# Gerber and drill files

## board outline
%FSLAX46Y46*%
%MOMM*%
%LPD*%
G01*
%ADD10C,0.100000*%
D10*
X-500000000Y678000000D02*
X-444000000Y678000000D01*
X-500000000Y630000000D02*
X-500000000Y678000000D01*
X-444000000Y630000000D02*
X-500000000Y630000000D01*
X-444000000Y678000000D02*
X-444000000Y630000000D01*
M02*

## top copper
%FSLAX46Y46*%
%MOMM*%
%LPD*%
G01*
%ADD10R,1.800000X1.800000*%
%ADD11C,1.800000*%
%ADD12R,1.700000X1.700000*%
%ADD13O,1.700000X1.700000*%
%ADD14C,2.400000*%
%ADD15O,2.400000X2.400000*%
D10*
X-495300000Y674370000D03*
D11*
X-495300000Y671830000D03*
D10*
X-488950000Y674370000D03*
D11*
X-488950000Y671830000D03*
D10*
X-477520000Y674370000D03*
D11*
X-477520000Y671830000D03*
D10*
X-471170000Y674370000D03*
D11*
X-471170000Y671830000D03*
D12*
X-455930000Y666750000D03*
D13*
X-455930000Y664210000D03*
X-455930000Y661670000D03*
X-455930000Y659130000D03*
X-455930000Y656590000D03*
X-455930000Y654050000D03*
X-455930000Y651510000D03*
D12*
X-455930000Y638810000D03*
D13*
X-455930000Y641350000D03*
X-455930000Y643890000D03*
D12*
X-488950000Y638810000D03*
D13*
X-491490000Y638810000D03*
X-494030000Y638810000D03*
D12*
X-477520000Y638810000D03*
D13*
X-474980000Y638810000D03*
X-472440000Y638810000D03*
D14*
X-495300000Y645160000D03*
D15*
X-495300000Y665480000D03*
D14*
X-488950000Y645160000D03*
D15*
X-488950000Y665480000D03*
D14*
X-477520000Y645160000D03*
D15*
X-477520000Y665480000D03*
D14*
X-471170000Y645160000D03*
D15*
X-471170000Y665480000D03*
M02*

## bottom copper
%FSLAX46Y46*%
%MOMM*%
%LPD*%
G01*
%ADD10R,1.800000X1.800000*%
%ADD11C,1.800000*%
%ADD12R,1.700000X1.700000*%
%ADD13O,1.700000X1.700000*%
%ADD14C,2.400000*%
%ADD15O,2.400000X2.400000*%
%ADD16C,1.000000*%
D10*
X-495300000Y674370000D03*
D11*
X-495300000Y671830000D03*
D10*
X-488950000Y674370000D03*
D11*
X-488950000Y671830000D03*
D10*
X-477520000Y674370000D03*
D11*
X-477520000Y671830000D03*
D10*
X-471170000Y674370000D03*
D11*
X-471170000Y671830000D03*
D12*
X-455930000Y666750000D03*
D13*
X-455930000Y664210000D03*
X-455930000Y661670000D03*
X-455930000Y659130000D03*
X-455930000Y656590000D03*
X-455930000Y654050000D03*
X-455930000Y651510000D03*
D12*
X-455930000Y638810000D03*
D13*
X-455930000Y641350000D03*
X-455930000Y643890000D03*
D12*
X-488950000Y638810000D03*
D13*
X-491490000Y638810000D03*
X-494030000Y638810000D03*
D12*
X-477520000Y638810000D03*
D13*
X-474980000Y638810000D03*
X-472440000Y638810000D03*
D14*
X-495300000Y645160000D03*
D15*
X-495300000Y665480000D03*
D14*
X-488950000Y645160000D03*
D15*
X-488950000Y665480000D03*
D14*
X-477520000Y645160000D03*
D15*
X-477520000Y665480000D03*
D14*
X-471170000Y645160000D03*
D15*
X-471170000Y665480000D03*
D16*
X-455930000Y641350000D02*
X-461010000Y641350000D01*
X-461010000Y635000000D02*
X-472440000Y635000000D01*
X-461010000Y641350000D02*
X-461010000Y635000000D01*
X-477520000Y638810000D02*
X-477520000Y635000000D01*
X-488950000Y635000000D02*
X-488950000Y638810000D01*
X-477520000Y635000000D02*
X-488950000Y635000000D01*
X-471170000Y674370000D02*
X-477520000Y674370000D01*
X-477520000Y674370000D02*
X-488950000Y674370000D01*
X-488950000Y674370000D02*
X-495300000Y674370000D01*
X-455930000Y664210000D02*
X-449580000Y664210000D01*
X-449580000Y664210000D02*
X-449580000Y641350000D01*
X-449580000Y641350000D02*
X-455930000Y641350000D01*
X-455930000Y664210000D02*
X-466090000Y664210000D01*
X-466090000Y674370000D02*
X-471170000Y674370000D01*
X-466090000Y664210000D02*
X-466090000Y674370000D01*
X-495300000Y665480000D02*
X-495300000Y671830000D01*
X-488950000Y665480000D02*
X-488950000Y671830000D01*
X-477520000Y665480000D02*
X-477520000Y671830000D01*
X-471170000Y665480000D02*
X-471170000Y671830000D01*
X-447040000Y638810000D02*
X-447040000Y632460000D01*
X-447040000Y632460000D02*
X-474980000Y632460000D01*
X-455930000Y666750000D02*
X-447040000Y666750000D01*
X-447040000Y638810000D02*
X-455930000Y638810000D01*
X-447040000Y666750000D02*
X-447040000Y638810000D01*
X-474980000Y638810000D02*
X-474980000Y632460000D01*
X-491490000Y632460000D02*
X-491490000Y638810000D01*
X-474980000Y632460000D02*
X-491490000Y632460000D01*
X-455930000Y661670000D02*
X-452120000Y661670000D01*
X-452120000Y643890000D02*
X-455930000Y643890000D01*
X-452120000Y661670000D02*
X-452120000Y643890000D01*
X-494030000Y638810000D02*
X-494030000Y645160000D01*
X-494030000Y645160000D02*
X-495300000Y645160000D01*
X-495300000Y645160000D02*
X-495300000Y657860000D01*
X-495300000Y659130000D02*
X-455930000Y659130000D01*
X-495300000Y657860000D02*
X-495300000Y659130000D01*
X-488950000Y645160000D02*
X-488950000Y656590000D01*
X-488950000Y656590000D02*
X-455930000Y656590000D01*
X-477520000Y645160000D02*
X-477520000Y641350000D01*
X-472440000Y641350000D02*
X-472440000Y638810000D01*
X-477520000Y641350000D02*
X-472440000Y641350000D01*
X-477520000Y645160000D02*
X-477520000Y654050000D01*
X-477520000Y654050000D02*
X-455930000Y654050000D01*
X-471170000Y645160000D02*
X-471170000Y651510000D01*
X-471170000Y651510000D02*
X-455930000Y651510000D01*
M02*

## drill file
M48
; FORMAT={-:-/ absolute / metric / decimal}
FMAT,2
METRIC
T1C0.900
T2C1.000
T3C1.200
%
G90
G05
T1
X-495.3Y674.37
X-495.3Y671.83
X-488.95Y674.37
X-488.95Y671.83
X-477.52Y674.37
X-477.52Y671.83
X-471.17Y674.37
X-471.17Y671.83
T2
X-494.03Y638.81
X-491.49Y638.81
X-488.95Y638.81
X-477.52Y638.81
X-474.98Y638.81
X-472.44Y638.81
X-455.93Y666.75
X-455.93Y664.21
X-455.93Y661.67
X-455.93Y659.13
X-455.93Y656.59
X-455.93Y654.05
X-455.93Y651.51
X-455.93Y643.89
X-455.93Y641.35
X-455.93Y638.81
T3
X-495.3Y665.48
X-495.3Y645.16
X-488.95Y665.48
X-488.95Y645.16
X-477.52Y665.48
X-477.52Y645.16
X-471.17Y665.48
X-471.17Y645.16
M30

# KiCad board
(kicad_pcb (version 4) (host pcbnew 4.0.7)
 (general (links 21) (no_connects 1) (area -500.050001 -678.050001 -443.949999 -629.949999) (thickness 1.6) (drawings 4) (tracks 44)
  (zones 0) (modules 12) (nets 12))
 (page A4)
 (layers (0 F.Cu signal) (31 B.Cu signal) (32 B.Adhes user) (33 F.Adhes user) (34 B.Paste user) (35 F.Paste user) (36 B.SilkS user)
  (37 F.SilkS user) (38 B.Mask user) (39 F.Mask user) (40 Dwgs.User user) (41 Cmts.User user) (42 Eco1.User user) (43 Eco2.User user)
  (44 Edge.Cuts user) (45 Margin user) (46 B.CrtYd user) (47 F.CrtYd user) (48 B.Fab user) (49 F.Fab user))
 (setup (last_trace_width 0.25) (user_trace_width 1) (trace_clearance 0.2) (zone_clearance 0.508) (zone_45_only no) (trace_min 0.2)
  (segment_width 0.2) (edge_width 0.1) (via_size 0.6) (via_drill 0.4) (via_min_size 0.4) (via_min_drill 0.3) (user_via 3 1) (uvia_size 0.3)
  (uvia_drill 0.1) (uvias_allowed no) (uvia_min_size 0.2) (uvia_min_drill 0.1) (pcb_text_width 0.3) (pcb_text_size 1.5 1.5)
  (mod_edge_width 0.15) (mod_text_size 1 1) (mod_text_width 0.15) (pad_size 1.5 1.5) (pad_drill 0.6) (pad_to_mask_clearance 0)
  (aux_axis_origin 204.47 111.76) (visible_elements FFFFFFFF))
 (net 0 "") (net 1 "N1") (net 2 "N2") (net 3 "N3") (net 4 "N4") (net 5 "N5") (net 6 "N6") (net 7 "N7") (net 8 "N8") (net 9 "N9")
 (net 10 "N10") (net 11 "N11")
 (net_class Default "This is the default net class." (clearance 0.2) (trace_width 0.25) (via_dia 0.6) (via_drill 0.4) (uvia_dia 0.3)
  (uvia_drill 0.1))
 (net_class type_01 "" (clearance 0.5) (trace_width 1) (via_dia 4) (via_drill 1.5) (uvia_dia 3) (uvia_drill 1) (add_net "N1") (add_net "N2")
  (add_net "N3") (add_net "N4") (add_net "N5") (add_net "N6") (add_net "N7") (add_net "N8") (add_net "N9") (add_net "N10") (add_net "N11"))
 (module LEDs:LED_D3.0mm (layer F.Cu) (at -495.3 -674.37 270)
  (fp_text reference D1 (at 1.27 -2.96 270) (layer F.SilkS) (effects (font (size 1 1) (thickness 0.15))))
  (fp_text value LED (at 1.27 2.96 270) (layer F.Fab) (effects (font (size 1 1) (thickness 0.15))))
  (pad 1 thru_hole rect (at 0 0 270) (size 1.8 1.8) (drill 0.9) (layers *.Cu *.Mask) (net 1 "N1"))
  (pad 2 thru_hole circle (at 2.54 0 270) (size 1.8 1.8) (drill 0.9) (layers *.Cu *.Mask) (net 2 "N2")))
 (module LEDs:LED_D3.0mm (layer F.Cu) (at -488.95 -674.37 270)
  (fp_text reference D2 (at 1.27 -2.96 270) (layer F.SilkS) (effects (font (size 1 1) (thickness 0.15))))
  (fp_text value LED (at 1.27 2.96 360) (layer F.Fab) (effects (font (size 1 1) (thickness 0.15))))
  (pad 1 thru_hole rect (at 0 0 270) (size 1.8 1.8) (drill 0.9) (layers *.Cu *.Mask) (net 1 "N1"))
  (pad 2 thru_hole circle (at 2.54 0 270) (size 1.8 1.8) (drill 0.9) (layers *.Cu *.Mask) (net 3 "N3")))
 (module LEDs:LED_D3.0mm (layer F.Cu) (at -477.52 -674.37 270)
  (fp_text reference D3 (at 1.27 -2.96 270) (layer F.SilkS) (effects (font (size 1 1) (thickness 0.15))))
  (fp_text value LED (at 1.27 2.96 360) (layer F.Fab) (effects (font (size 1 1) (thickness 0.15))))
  (pad 1 thru_hole rect (at 0 0 270) (size 1.8 1.8) (drill 0.9) (layers *.Cu *.Mask) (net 1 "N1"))
  (pad 2 thru_hole circle (at 2.54 0 270) (size 1.8 1.8) (drill 0.9) (layers *.Cu *.Mask) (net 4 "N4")))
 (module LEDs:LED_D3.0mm (layer F.Cu) (at -471.17 -674.37 270)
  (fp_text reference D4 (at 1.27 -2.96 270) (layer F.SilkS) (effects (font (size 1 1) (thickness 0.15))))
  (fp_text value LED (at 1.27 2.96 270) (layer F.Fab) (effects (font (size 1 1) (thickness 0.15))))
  (pad 1 thru_hole rect (at 0 0 270) (size 1.8 1.8) (drill 0.9) (layers *.Cu *.Mask) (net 1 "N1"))
  (pad 2 thru_hole circle (at 2.54 0 270) (size 1.8 1.8) (drill 0.9) (layers *.Cu *.Mask) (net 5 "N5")))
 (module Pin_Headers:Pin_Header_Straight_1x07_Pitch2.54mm (layer F.Cu) (at -455.93 -666.75)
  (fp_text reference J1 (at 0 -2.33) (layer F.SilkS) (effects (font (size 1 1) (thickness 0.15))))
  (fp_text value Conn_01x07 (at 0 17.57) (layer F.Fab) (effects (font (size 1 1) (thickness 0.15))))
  (pad 1 thru_hole rect (at 0 0) (size 1.7 1.7) (drill 1) (layers *.Cu *.Mask) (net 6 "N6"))
  (pad 2 thru_hole oval (at 0 2.54) (size 1.7 1.7) (drill 1) (layers *.Cu *.Mask) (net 1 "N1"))
  (pad 3 thru_hole oval (at 0 5.08) (size 1.7 1.7) (drill 1) (layers *.Cu *.Mask) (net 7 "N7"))
  (pad 4 thru_hole oval (at 0 7.62) (size 1.7 1.7) (drill 1) (layers *.Cu *.Mask) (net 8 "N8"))
  (pad 5 thru_hole oval (at 0 10.16) (size 1.7 1.7) (drill 1) (layers *.Cu *.Mask) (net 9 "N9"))
  (pad 6 thru_hole oval (at 0 12.7) (size 1.7 1.7) (drill 1) (layers *.Cu *.Mask) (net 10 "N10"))
  (pad 7 thru_hole oval (at 0 15.24) (size 1.7 1.7) (drill 1) (layers *.Cu *.Mask) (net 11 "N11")))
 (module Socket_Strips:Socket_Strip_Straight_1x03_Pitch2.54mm (layer F.Cu) (at -455.93 -638.81 180)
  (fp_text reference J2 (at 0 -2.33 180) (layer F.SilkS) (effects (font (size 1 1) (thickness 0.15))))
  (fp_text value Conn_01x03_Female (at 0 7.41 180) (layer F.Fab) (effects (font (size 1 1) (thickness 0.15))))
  (pad 1 thru_hole rect (at 0 0 180) (size 1.7 1.7) (drill 1) (layers *.Cu *.Mask) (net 6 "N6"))
  (pad 2 thru_hole oval (at 0 2.54 180) (size 1.7 1.7) (drill 1) (layers *.Cu *.Mask) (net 1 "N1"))
  (pad 3 thru_hole oval (at 0 5.08 180) (size 1.7 1.7) (drill 1) (layers *.Cu *.Mask) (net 7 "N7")))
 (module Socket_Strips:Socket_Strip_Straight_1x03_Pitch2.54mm (layer F.Cu) (at -488.95 -638.81 270)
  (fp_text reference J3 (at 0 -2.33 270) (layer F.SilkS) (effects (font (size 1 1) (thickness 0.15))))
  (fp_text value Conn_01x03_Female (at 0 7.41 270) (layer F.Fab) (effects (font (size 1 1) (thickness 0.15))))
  (pad 1 thru_hole rect (at 0 0 270) (size 1.7 1.7) (drill 1) (layers *.Cu *.Mask) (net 1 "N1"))
  (pad 2 thru_hole oval (at 0 2.54 270) (size 1.7 1.7) (drill 1) (layers *.Cu *.Mask) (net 6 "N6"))
  (pad 3 thru_hole oval (at 0 5.08 270) (size 1.7 1.7) (drill 1) (layers *.Cu *.Mask) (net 8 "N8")))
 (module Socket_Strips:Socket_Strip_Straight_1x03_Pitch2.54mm (layer F.Cu) (at -477.52 -638.81 90)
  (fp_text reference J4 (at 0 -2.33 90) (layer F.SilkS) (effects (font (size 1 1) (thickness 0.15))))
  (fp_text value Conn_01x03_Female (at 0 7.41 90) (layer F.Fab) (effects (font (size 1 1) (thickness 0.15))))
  (pad 1 thru_hole rect (at 0 0 90) (size 1.7 1.7) (drill 1) (layers *.Cu *.Mask) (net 1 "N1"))
  (pad 2 thru_hole oval (at 0 2.54 90) (size 1.7 1.7) (drill 1) (layers *.Cu *.Mask) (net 6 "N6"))
  (pad 3 thru_hole oval (at 0 5.08 90) (size 1.7 1.7) (drill 1) (layers *.Cu *.Mask) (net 10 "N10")))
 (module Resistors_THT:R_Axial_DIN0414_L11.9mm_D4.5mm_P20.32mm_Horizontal (layer F.Cu) (at -495.3 -645.16 90)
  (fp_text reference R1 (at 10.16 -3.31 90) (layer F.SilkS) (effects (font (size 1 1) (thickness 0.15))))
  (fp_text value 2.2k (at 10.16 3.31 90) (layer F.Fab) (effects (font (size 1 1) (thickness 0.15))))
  (pad 1 thru_hole circle (at 0 0 90) (size 2.4 2.4) (drill 1.2) (layers *.Cu *.Mask) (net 8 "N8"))
  (pad 2 thru_hole oval (at 20.32 0 90) (size 2.4 2.4) (drill 1.2) (layers *.Cu *.Mask) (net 2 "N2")))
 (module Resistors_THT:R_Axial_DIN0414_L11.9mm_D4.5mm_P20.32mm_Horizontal (layer F.Cu) (at -488.95 -645.16 90)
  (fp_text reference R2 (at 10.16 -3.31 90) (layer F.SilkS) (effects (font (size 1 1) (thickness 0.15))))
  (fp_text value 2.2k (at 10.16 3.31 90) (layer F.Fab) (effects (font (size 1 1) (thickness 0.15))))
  (pad 1 thru_hole circle (at 0 0 90) (size 2.4 2.4) (drill 1.2) (layers *.Cu *.Mask) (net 9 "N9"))
  (pad 2 thru_hole oval (at 20.32 0 90) (size 2.4 2.4) (drill 1.2) (layers *.Cu *.Mask) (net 3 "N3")))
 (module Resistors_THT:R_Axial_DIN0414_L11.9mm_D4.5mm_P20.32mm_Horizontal (layer F.Cu) (at -477.52 -645.16 90)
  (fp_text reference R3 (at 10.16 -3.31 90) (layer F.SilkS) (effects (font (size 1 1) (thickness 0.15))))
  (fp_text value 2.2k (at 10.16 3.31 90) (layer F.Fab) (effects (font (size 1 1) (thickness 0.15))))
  (pad 1 thru_hole circle (at 0 0 90) (size 2.4 2.4) (drill 1.2) (layers *.Cu *.Mask) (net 10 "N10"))
  (pad 2 thru_hole oval (at 20.32 0 90) (size 2.4 2.4) (drill 1.2) (layers *.Cu *.Mask) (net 4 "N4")))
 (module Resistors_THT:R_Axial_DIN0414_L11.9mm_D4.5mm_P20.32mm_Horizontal (layer F.Cu) (at -471.17 -645.16 90)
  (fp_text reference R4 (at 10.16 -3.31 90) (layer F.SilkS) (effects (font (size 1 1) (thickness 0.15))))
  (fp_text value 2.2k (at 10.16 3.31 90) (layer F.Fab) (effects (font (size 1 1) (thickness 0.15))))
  (pad 1 thru_hole circle (at 0 0 90) (size 2.4 2.4) (drill 1.2) (layers *.Cu *.Mask) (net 11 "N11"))
  (pad 2 thru_hole oval (at 20.32 0 90) (size 2.4 2.4) (drill 1.2) (layers *.Cu *.Mask) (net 5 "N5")))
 (gr_line (start -500 -678) (end -444 -678) (angle 90) (layer Edge.Cuts) (width 0.1))
 (gr_line (start -500 -630) (end -500 -678) (angle 90) (layer Edge.Cuts) (width 0.1))
 (gr_line (start -444 -630) (end -500 -630) (angle 90) (layer Edge.Cuts) (width 0.1))
 (gr_line (start -444 -678) (end -444 -630) (angle 90) (layer Edge.Cuts) (width 0.1))
 (segment (start -455.93 -641.35) (end -461.01 -641.35) (width 1) (layer B.Cu) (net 1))
 (segment (start -461.01 -635) (end -472.44 -635) (width 1) (layer B.Cu) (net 1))
 (segment (start -461.01 -641.35) (end -461.01 -635) (width 1) (layer B.Cu) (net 1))
 (segment (start -477.52 -638.81) (end -477.52 -635) (width 1) (layer B.Cu) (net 1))
 (segment (start -488.95 -635) (end -488.95 -638.81) (width 1) (layer B.Cu) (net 1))
 (segment (start -477.52 -635) (end -488.95 -635) (width 1) (layer B.Cu) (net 1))
 (segment (start -471.17 -674.37) (end -477.52 -674.37) (width 1) (layer B.Cu) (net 1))
 (segment (start -477.52 -674.37) (end -488.95 -674.37) (width 1) (layer B.Cu) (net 1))
 (segment (start -488.95 -674.37) (end -495.3 -674.37) (width 1) (layer B.Cu) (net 1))
 (segment (start -455.93 -664.21) (end -449.58 -664.21) (width 1) (layer B.Cu) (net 1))
 (segment (start -449.58 -664.21) (end -449.58 -641.35) (width 1) (layer B.Cu) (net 1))
 (segment (start -449.58 -641.35) (end -455.93 -641.35) (width 1) (layer B.Cu) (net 1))
 (segment (start -455.93 -664.21) (end -466.09 -664.21) (width 1) (layer B.Cu) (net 1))
 (segment (start -466.09 -674.37) (end -471.17 -674.37) (width 1) (layer B.Cu) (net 1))
 (segment (start -466.09 -664.21) (end -466.09 -674.37) (width 1) (layer B.Cu) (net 1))
 (segment (start -495.3 -665.48) (end -495.3 -671.83) (width 1) (layer B.Cu) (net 2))
 (segment (start -488.95 -665.48) (end -488.95 -671.83) (width 1) (layer B.Cu) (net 3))
 (segment (start -477.52 -665.48) (end -477.52 -671.83) (width 1) (layer B.Cu) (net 4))
 (segment (start -471.17 -665.48) (end -471.17 -671.83) (width 1) (layer B.Cu) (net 5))
 (segment (start -447.04 -638.81) (end -447.04 -632.46) (width 1) (layer B.Cu) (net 6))
 (segment (start -447.04 -632.46) (end -474.98 -632.46) (width 1) (layer B.Cu) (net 6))
 (segment (start -455.93 -666.75) (end -447.04 -666.75) (width 1) (layer B.Cu) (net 6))
 (segment (start -447.04 -638.81) (end -455.93 -638.81) (width 1) (layer B.Cu) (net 6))
 (segment (start -447.04 -666.75) (end -447.04 -638.81) (width 1) (layer B.Cu) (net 6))
 (segment (start -474.98 -638.81) (end -474.98 -632.46) (width 1) (layer B.Cu) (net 6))
 (segment (start -491.49 -632.46) (end -491.49 -638.81) (width 1) (layer B.Cu) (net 6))
 (segment (start -474.98 -632.46) (end -491.49 -632.46) (width 1) (layer B.Cu) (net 6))
 (segment (start -455.93 -661.67) (end -452.12 -661.67) (width 1) (layer B.Cu) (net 7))
 (segment (start -452.12 -643.89) (end -455.93 -643.89) (width 1) (layer B.Cu) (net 7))
 (segment (start -452.12 -661.67) (end -452.12 -643.89) (width 1) (layer B.Cu) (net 7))
 (segment (start -494.03 -638.81) (end -494.03 -645.16) (width 1) (layer B.Cu) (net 8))
 (segment (start -494.03 -645.16) (end -495.3 -645.16) (width 1) (layer B.Cu) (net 8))
 (segment (start -495.3 -645.16) (end -495.3 -657.86) (width 1) (layer B.Cu) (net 8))
 (segment (start -495.3 -659.13) (end -455.93 -659.13) (width 1) (layer B.Cu) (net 8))
 (segment (start -495.3 -657.86) (end -495.3 -659.13) (width 1) (layer B.Cu) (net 8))
 (segment (start -488.95 -645.16) (end -488.95 -656.59) (width 1) (layer B.Cu) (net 9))
 (segment (start -488.95 -656.59) (end -455.93 -656.59) (width 1) (layer B.Cu) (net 9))
 (segment (start -477.52 -645.16) (end -477.52 -641.35) (width 1) (layer B.Cu) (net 10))
 (segment (start -472.44 -641.35) (end -472.44 -638.81) (width 1) (layer B.Cu) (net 10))
 (segment (start -477.52 -641.35) (end -472.44 -641.35) (width 1) (layer B.Cu) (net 10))
 (segment (start -477.52 -645.16) (end -477.52 -654.05) (width 1) (layer B.Cu) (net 10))
 (segment (start -477.52 -654.05) (end -455.93 -654.05) (width 1) (layer B.Cu) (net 10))
 (segment (start -471.17 -645.16) (end -471.17 -651.51) (width 1) (layer B.Cu) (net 11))
 (segment (start -471.17 -651.51) (end -455.93 -651.51) (width 1) (layer B.Cu) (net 11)))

